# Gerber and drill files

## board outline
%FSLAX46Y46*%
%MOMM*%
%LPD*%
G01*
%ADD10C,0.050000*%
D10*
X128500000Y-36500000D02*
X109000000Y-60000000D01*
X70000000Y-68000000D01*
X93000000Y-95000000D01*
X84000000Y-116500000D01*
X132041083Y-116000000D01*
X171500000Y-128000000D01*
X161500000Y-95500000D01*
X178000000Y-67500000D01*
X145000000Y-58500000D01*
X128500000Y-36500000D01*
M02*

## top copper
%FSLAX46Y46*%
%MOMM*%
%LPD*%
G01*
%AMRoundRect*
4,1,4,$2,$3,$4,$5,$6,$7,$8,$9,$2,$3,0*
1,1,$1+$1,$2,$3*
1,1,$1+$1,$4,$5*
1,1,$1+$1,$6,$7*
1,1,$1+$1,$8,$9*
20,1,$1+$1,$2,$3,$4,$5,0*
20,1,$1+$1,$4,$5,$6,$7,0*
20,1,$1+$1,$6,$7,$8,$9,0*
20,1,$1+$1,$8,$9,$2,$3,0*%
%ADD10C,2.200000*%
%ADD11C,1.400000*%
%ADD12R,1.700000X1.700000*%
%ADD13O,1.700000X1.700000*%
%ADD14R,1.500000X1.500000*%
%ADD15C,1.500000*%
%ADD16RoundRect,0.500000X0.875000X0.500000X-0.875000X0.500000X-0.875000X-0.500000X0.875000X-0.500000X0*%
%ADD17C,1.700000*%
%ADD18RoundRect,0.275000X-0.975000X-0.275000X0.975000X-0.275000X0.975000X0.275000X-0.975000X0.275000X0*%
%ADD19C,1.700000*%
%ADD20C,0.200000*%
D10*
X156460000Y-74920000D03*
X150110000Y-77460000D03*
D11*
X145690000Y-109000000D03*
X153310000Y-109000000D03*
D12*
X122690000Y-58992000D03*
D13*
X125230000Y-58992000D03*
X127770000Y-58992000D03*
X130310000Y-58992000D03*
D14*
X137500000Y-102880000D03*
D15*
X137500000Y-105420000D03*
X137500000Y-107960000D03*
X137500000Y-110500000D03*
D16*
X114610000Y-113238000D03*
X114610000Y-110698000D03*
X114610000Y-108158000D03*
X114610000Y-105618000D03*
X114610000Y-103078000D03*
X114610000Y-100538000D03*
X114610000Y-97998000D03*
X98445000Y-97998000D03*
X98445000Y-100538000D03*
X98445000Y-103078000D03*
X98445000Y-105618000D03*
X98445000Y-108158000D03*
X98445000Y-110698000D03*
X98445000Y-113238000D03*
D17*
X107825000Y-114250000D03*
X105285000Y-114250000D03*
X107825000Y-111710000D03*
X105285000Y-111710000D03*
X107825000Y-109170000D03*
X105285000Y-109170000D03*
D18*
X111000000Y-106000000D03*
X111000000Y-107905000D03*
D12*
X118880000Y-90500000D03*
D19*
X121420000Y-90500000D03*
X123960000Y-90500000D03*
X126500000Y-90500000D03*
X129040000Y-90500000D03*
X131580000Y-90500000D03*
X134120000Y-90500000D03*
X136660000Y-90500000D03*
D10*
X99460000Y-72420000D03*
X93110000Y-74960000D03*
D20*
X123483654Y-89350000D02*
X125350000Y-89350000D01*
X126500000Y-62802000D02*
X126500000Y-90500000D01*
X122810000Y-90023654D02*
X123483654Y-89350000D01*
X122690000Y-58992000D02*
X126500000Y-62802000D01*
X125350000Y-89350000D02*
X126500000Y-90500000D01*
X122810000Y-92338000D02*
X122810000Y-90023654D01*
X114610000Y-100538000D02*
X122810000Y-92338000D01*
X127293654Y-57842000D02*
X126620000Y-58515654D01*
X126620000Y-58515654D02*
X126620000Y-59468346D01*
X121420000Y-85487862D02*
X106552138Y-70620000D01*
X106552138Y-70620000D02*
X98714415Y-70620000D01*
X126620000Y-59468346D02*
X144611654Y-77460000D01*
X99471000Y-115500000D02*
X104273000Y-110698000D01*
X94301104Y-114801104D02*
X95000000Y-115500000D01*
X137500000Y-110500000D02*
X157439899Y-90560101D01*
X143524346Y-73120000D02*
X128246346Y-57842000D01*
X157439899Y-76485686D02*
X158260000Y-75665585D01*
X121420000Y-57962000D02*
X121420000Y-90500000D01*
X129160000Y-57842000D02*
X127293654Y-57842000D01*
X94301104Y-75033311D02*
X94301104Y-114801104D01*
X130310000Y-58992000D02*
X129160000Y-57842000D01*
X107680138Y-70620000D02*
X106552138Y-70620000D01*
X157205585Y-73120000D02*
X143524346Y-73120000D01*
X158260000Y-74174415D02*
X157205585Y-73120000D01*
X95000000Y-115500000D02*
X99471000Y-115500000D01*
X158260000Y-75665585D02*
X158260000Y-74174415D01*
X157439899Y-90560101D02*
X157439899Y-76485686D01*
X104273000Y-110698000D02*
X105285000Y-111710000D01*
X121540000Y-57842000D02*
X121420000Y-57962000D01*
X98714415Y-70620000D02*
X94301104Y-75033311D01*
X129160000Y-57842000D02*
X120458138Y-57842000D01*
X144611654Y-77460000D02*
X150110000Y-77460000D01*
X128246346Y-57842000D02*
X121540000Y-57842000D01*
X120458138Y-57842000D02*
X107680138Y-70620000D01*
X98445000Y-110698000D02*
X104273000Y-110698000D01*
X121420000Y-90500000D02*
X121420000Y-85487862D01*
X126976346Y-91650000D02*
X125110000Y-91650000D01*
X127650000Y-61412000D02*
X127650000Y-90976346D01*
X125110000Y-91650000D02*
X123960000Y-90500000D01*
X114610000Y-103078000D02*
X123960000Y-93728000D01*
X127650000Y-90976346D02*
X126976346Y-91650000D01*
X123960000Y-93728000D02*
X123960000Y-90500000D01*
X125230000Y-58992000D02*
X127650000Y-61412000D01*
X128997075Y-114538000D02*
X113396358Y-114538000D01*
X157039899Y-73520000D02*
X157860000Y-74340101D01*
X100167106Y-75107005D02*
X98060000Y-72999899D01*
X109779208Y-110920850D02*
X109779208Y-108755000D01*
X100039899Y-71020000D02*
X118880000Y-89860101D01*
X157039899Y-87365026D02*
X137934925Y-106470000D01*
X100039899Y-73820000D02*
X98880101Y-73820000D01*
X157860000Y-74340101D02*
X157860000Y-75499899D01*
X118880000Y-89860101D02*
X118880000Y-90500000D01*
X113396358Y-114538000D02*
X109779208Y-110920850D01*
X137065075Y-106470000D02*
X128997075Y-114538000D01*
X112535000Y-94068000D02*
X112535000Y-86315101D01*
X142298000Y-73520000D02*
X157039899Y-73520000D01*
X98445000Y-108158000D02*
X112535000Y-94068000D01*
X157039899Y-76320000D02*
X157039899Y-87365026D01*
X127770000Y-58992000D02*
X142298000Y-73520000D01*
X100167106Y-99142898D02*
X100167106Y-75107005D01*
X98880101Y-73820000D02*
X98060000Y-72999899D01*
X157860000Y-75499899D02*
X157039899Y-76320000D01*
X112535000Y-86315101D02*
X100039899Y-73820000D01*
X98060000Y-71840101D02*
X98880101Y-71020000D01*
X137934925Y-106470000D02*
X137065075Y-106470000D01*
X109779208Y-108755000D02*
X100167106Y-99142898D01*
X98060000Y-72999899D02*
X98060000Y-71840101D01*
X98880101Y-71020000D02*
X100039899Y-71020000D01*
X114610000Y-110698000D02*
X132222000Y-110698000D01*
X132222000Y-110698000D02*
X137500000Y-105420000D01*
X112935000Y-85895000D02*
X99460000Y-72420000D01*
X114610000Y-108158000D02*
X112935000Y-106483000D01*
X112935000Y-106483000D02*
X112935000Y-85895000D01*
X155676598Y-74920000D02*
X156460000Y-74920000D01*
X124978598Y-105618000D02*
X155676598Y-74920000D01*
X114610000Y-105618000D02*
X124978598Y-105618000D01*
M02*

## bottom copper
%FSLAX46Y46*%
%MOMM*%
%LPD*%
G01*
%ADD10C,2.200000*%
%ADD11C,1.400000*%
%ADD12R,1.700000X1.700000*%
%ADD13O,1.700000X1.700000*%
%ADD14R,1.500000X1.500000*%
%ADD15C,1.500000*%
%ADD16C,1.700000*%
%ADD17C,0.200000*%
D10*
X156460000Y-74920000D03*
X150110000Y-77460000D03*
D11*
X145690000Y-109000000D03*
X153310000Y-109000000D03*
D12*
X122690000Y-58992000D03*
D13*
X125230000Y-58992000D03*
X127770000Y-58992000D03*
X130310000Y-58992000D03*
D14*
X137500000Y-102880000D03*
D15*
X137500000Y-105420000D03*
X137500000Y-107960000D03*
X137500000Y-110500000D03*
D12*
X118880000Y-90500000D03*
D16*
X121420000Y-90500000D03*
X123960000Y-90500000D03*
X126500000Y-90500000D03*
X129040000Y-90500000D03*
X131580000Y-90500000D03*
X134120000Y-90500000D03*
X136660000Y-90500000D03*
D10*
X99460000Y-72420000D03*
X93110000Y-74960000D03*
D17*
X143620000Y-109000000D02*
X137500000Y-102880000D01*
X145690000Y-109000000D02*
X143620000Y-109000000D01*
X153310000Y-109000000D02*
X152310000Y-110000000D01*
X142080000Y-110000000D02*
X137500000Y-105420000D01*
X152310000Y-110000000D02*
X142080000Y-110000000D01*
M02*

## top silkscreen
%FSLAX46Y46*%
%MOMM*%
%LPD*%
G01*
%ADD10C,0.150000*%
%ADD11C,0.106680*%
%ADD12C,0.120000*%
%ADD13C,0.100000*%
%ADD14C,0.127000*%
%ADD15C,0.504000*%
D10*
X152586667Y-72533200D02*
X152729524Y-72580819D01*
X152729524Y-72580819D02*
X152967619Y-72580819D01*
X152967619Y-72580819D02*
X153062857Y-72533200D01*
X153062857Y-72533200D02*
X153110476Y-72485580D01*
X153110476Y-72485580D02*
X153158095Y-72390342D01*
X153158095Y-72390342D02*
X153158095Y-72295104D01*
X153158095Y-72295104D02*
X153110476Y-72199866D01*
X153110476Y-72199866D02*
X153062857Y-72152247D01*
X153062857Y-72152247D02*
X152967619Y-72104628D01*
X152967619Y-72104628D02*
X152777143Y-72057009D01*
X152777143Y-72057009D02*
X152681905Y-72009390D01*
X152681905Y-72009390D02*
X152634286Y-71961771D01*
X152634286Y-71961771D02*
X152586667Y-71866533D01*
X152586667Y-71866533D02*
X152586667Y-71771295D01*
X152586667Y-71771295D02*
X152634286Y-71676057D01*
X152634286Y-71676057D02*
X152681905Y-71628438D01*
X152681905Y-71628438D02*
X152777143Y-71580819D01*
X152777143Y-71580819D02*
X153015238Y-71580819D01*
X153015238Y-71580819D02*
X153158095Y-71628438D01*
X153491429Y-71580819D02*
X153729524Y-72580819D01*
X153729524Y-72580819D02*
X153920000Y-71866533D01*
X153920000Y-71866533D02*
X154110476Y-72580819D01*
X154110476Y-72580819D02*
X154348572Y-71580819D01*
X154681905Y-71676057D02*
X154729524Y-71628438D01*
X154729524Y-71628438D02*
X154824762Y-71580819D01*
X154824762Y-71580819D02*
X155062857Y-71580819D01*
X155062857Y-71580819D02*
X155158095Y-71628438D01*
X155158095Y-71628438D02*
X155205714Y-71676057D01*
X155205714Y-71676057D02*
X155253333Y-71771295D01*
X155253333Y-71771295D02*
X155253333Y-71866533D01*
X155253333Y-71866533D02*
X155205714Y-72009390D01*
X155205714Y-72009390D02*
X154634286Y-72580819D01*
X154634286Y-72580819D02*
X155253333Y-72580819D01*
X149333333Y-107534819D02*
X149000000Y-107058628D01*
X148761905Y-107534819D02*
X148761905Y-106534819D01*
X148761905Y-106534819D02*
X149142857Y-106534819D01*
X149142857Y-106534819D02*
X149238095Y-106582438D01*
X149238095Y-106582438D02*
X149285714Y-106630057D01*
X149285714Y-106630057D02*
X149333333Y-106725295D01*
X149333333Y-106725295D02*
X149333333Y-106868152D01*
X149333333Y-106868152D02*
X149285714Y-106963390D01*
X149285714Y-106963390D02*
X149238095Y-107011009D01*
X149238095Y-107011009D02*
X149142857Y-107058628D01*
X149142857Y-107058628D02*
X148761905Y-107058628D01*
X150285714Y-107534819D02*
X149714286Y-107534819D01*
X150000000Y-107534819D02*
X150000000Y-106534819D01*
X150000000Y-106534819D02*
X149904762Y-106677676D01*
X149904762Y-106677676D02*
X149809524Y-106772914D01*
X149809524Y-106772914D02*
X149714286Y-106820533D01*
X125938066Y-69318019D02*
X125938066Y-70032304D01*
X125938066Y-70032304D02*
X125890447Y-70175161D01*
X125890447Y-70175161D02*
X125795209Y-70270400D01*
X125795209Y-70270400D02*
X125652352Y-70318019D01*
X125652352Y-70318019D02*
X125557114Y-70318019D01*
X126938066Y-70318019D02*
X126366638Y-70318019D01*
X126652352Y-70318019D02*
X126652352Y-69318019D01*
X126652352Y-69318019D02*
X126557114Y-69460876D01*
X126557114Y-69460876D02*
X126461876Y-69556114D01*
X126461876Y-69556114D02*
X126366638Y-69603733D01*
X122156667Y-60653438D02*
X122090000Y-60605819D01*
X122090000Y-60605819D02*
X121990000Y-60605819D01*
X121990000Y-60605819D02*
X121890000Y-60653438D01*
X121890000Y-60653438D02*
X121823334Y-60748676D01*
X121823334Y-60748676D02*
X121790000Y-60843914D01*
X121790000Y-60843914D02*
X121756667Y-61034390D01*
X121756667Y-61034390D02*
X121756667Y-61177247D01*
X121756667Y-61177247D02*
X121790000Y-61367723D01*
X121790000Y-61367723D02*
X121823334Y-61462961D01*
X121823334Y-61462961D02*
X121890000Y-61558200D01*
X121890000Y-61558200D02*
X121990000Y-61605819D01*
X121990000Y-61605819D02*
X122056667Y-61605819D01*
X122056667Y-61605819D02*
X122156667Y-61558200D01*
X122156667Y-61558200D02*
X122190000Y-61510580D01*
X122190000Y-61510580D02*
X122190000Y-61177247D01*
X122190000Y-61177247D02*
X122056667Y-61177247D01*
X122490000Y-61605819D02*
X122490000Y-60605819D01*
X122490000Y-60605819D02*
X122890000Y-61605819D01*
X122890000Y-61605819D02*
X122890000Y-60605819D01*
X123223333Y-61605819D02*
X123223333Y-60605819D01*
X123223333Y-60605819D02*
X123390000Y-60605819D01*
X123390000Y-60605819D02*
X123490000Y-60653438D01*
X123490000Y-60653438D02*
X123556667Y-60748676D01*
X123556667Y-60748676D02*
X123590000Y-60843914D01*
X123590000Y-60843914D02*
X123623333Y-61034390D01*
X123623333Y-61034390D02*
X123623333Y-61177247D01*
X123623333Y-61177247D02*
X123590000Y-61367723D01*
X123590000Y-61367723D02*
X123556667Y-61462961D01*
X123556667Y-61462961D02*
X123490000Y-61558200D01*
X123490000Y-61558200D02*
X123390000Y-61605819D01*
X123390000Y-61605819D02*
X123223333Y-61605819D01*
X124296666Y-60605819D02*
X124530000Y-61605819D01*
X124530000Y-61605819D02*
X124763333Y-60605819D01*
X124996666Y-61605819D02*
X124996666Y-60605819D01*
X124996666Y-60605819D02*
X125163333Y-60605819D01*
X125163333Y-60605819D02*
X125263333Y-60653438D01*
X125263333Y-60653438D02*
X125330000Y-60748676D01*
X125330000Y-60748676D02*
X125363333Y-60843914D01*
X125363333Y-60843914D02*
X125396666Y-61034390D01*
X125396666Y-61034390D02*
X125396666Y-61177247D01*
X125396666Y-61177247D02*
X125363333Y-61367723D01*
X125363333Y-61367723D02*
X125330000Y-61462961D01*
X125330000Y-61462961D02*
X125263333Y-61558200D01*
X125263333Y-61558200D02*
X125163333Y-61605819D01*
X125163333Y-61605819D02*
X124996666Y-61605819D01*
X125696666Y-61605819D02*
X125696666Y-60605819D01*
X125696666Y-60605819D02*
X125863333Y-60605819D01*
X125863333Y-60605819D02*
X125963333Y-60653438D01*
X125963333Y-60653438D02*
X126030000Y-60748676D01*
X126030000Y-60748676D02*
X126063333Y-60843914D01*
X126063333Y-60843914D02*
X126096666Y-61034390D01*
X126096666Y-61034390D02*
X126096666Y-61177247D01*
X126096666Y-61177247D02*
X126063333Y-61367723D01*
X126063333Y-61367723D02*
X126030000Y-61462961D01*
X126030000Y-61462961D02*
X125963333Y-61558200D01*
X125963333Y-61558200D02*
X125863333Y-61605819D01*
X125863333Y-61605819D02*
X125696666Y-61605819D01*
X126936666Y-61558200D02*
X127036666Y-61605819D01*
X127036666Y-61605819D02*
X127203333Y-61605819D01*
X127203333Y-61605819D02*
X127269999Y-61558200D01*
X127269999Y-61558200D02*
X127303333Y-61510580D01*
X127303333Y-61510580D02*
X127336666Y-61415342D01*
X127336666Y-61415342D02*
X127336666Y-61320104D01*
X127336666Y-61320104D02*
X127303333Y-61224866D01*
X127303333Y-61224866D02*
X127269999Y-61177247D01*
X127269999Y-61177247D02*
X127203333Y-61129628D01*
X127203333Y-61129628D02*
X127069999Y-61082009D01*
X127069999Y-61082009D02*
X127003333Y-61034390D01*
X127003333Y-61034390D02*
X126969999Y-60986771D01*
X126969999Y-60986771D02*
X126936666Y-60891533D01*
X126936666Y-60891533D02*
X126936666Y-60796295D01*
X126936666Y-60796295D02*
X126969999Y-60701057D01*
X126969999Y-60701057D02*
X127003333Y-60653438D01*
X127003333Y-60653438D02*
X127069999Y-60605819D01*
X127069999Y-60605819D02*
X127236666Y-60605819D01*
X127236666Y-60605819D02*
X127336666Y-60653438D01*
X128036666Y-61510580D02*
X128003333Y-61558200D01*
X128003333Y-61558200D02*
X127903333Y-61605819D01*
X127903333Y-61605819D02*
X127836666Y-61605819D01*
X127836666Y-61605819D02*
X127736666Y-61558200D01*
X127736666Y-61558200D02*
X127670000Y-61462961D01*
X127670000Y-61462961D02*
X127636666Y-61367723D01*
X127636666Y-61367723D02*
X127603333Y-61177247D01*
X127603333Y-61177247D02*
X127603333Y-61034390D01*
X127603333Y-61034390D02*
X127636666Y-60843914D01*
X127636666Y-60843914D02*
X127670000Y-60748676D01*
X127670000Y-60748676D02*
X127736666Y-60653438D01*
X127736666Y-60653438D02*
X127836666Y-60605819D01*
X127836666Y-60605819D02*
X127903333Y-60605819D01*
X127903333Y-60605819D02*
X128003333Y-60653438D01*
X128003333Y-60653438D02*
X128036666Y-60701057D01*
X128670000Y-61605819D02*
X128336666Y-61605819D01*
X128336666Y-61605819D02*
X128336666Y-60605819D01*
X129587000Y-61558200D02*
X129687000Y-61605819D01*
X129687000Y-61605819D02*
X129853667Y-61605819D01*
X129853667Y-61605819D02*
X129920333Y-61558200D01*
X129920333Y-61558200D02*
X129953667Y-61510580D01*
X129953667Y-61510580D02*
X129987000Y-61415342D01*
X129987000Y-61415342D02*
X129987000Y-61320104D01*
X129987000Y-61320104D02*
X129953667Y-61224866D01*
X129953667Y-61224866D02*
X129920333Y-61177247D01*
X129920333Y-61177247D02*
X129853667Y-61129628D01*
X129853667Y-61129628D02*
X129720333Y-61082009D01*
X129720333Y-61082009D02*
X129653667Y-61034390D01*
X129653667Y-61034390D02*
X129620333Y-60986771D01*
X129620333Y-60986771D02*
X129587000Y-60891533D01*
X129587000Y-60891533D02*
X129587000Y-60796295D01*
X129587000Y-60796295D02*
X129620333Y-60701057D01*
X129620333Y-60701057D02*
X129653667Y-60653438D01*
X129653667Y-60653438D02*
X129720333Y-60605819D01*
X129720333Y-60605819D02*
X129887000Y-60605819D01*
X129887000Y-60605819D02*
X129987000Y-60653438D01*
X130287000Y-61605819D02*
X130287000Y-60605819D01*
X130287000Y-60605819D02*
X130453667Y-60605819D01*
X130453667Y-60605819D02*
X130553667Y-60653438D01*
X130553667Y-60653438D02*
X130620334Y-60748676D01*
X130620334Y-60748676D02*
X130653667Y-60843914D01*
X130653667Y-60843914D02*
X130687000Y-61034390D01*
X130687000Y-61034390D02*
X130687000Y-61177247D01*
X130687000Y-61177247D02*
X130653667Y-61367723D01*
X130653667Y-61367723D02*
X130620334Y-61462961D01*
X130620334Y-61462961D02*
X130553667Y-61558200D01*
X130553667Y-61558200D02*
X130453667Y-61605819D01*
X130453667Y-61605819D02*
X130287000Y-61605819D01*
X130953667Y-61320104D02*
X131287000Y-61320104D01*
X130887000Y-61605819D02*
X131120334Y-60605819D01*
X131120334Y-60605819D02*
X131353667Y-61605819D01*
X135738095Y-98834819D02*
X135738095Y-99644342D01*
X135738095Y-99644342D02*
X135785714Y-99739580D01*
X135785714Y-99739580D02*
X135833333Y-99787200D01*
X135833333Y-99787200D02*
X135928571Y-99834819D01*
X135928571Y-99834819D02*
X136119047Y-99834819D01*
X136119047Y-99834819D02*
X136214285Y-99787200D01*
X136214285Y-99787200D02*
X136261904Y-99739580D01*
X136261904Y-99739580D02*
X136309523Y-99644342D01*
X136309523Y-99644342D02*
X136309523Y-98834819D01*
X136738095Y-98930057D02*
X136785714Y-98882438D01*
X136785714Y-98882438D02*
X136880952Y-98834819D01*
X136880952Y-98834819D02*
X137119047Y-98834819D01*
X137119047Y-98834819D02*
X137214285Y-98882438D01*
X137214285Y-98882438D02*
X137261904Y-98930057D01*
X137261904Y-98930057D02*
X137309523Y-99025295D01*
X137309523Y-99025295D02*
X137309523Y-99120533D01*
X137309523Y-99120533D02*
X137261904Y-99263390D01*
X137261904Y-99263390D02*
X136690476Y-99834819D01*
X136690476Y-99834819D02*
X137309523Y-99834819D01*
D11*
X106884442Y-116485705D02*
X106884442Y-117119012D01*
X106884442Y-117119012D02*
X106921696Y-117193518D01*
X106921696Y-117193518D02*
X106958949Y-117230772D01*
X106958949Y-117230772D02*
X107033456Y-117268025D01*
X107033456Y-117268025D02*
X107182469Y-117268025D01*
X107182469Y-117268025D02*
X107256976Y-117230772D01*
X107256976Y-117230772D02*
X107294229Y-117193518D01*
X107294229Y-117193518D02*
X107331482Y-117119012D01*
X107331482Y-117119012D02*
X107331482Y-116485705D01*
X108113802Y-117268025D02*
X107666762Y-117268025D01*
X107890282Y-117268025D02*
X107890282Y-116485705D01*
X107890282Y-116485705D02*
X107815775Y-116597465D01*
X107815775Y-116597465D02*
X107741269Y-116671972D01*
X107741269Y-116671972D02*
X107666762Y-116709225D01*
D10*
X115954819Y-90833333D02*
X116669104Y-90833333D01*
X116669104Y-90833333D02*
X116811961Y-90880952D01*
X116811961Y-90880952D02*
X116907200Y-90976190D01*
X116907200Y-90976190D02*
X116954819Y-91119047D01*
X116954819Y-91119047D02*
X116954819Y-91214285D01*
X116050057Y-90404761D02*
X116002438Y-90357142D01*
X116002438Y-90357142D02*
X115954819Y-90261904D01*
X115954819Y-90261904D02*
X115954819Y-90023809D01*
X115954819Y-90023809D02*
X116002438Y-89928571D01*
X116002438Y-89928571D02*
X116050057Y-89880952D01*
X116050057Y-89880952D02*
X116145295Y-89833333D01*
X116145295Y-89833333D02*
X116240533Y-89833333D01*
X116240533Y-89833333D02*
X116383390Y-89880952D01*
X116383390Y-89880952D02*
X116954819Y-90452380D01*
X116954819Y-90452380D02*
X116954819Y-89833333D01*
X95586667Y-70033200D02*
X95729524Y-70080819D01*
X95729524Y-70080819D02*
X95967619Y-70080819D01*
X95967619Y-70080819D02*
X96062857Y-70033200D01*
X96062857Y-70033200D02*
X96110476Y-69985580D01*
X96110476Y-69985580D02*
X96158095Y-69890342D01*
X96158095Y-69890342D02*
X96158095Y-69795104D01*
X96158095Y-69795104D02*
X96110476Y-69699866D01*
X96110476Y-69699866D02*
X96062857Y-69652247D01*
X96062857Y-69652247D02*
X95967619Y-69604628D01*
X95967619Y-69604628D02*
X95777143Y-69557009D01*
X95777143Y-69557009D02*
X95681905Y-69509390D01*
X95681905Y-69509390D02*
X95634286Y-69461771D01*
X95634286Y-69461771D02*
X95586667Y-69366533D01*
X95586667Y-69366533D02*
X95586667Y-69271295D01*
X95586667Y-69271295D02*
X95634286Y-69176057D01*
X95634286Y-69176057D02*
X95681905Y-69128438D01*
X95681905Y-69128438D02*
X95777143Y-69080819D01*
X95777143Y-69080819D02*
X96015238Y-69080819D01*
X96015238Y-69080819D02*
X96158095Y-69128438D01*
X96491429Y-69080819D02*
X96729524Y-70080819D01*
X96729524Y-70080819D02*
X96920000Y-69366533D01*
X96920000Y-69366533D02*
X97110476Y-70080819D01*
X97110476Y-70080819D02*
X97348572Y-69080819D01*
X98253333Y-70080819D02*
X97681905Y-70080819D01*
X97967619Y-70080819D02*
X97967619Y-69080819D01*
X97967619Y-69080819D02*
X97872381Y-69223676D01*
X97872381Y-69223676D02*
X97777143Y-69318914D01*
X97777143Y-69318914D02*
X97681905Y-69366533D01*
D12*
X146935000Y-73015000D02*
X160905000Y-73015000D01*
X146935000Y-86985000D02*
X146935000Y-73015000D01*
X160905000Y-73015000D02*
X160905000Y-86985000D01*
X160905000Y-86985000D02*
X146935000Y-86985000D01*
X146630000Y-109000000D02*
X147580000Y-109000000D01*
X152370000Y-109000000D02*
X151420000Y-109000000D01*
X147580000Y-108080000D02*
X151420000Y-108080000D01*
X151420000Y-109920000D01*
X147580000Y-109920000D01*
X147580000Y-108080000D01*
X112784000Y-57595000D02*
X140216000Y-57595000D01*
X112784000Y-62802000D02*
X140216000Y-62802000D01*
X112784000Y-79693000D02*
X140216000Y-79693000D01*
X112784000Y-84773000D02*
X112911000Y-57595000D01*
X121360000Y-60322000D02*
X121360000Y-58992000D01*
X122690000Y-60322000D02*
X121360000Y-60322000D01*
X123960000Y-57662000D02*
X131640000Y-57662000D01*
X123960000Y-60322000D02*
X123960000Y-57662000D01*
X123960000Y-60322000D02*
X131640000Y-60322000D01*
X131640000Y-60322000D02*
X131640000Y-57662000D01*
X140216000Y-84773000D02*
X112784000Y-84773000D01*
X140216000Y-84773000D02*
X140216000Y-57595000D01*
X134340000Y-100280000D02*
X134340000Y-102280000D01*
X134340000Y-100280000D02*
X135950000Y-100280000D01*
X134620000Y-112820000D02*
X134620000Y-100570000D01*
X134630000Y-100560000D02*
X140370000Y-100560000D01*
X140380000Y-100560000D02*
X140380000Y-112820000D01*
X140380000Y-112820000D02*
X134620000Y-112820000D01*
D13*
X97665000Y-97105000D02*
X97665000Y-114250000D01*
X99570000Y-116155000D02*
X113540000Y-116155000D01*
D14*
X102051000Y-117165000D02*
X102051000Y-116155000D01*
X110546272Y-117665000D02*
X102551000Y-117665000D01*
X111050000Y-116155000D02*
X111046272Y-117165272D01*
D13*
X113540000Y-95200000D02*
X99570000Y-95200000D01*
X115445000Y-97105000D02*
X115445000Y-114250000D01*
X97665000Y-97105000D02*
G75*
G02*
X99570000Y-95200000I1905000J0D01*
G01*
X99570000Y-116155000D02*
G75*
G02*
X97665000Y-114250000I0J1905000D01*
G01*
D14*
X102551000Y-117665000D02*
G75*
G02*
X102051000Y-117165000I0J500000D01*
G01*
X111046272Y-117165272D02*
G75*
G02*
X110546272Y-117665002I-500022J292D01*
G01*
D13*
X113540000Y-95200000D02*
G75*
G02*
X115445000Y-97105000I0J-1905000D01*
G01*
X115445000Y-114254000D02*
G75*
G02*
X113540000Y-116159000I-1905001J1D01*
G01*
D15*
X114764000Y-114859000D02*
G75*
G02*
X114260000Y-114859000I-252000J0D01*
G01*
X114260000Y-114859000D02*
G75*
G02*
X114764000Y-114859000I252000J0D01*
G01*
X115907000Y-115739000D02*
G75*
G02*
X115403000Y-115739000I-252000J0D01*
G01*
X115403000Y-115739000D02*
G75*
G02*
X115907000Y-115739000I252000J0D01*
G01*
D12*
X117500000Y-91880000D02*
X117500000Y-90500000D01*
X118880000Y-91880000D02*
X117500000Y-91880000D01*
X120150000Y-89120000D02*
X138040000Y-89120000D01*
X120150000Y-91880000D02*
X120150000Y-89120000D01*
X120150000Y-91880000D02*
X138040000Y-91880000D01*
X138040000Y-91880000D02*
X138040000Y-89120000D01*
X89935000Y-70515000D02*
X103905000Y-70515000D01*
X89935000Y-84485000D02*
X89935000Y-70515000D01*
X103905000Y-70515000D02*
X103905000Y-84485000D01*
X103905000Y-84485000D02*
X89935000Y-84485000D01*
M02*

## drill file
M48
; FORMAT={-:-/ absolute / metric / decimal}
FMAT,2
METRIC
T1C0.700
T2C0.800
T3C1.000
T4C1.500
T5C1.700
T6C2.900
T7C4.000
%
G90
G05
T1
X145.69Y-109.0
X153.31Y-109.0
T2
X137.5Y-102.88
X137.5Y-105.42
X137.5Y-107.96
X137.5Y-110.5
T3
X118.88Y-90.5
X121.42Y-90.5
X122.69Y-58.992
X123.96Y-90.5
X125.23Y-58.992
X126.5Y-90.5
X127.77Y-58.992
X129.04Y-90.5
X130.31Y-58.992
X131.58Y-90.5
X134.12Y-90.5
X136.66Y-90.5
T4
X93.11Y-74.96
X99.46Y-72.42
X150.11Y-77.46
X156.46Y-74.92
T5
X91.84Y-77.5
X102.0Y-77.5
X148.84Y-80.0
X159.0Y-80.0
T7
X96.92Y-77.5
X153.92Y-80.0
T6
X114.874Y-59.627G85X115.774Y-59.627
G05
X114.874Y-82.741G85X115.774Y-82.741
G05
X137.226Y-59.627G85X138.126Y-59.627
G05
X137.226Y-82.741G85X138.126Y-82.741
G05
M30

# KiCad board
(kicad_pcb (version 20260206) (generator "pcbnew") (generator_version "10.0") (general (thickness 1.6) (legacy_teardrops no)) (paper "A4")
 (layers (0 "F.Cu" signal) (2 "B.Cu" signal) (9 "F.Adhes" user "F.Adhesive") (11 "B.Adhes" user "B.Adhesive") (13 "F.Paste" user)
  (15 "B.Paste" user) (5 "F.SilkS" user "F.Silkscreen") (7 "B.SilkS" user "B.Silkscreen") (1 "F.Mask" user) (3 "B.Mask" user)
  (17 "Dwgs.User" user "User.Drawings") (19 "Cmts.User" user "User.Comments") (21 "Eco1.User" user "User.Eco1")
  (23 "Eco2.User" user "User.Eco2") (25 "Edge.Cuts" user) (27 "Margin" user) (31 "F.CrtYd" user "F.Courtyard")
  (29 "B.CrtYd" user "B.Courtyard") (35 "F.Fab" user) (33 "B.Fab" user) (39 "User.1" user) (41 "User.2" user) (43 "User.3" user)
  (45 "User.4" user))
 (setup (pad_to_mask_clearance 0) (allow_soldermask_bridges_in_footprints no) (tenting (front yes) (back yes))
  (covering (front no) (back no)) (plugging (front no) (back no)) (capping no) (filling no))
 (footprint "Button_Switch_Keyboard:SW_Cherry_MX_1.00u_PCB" (layer "F.Cu") (at 156.46 74.92)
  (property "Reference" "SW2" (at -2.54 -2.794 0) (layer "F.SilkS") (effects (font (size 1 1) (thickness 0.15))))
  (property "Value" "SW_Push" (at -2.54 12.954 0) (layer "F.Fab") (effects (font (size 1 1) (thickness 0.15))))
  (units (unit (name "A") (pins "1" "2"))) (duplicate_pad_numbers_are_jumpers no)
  (fp_line (start -9.525 -1.905) (end 4.445 -1.905) (stroke (width 0.12) (type solid)) (layer "F.SilkS"))
  (fp_line (start -9.525 12.065) (end -9.525 -1.905) (stroke (width 0.12) (type solid)) (layer "F.SilkS"))
  (fp_line (start 4.445 -1.905) (end 4.445 12.065) (stroke (width 0.12) (type solid)) (layer "F.SilkS"))
  (fp_line (start 4.445 12.065) (end -9.525 12.065) (stroke (width 0.12) (type solid)) (layer "F.SilkS"))
  (pad "" np_thru_hole circle (at -7.62 5.08) (size 1.7 1.7) (drill 1.7) (layers "*.Cu" "*.Mask"))
  (pad "" np_thru_hole circle (at -2.54 5.08) (size 4 4) (drill 4) (layers "*.Cu" "*.Mask"))
  (pad "" np_thru_hole circle (at 2.54 5.08) (size 1.7 1.7) (drill 1.7) (layers "*.Cu" "*.Mask"))
  (pad "1" thru_hole circle (at 0 0) (size 2.2 2.2) (drill 1.5) (layers "*.Cu" "*.Mask") (remove_unused_layers no) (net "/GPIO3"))
  (pad "2" thru_hole circle (at -6.35 2.54) (size 2.2 2.2) (drill 1.5) (layers "*.Cu" "*.Mask") (remove_unused_layers no) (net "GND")))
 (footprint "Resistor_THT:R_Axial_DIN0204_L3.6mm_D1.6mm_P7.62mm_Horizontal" (layer "F.Cu") (at 145.69 109)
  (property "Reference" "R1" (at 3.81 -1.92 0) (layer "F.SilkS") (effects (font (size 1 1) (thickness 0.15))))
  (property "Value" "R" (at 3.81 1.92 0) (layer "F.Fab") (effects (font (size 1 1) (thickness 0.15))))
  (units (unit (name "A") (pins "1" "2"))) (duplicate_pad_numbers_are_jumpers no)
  (fp_line (start 0.94 0) (end 1.89 0) (stroke (width 0.12) (type solid)) (layer "F.SilkS"))
  (fp_line (start 6.68 0) (end 5.73 0) (stroke (width 0.12) (type solid)) (layer "F.SilkS"))
  (fp_rect (start 1.89 -0.92) (end 5.73 0.92) (stroke (width 0.12) (type solid)) (fill no) (layer "F.SilkS"))
  (pad "1" thru_hole circle (at 0 0) (size 1.4 1.4) (drill 0.7) (layers "*.Cu" "*.Mask") (remove_unused_layers no) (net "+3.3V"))
  (pad "2" thru_hole circle (at 7.62 0) (size 1.4 1.4) (drill 0.7) (layers "*.Cu" "*.Mask") (remove_unused_layers no) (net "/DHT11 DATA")))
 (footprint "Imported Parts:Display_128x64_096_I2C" (layer "F.Cu") (at 126.5 58.992)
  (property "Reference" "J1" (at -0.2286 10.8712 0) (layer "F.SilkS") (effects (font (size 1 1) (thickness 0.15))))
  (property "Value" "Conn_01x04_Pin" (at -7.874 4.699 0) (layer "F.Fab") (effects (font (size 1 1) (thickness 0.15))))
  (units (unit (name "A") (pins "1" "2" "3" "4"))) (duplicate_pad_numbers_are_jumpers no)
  (fp_line (start -13.716 -1.397) (end 13.716 -1.397) (stroke (width 0.12) (type solid)) (layer "F.SilkS"))
  (fp_line (start -13.716 3.81) (end 13.716 3.81) (stroke (width 0.12) (type solid)) (layer "F.SilkS"))
  (fp_line (start -13.716 20.701) (end 13.716 20.701) (stroke (width 0.12) (type solid)) (layer "F.SilkS"))
  (fp_line (start -13.716 25.781) (end -13.589 -1.397) (stroke (width 0.12) (type solid)) (layer "F.SilkS"))
  (fp_line (start -5.14 1.33) (end -5.14 0) (stroke (width 0.12) (type solid)) (layer "F.SilkS"))
  (fp_line (start -3.81 1.33) (end -5.14 1.33) (stroke (width 0.12) (type solid)) (layer "F.SilkS"))
  (fp_line (start -2.54 -1.33) (end 5.14 -1.33) (stroke (width 0.12) (type solid)) (layer "F.SilkS"))
  (fp_line (start -2.54 1.33) (end -2.54 -1.33) (stroke (width 0.12) (type solid)) (layer "F.SilkS"))
  (fp_line (start -2.54 1.33) (end 5.14 1.33) (stroke (width 0.12) (type solid)) (layer "F.SilkS"))
  (fp_line (start 5.14 1.33) (end 5.14 -1.33) (stroke (width 0.12) (type solid)) (layer "F.SilkS"))
  (fp_line (start 13.716 25.781) (end -13.716 25.781) (stroke (width 0.12) (type solid)) (layer "F.SilkS"))
  (fp_line (start 13.716 25.781) (end 13.716 -1.397) (stroke (width 0.12) (type solid)) (layer "F.SilkS"))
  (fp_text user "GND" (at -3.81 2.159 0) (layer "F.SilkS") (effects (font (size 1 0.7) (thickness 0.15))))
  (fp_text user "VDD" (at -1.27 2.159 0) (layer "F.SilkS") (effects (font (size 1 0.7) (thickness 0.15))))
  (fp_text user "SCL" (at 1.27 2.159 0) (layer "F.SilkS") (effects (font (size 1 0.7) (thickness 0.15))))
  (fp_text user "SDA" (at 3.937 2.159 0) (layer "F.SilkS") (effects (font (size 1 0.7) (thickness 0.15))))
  (pad "" np_thru_hole oval (at -11.176 0.635) (size 3.8 2.9) (drill oval 3.8 2.9) (layers "*.Cu" "*.Mask"))
  (pad "" np_thru_hole oval (at -11.176 23.749) (size 3.8 2.9) (drill oval 3.8 2.9) (layers "*.Cu" "*.Mask"))
  (pad "" np_thru_hole oval (at 11.176 0.635) (size 3.8 2.9) (drill oval 3.8 2.9) (layers "*.Cu" "*.Mask"))
  (pad "" np_thru_hole oval (at 11.176 23.749) (size 3.8 2.9) (drill oval 3.8 2.9) (layers "*.Cu" "*.Mask"))
  (pad "1" thru_hole rect (at -3.81 0 90) (size 1.7 1.7) (drill 1) (layers "*.Cu" "*.Mask") (remove_unused_layers no) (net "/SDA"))
  (pad "2" thru_hole oval (at -1.27 0 90) (size 1.7 1.7) (drill 1) (layers "*.Cu" "*.Mask") (remove_unused_layers no) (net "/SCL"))
  (pad "3" thru_hole oval (at 1.27 0 90) (size 1.7 1.7) (drill 1) (layers "*.Cu" "*.Mask") (remove_unused_layers no) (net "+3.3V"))
  (pad "4" thru_hole oval (at 3.81 0 90) (size 1.7 1.7) (drill 1) (layers "*.Cu" "*.Mask") (remove_unused_layers no) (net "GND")))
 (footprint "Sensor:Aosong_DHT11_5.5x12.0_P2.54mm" (layer "F.Cu") (at 137.5 102.88)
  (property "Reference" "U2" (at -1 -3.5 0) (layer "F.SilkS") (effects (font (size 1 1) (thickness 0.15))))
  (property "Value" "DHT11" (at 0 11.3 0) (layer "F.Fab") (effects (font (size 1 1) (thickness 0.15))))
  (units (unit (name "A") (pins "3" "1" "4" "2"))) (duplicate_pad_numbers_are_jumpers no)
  (fp_line (start -3.16 -2.6) (end -3.16 -0.6) (stroke (width 0.12) (type solid)) (layer "F.SilkS"))
  (fp_line (start -3.16 -2.6) (end -1.55 -2.6) (stroke (width 0.12) (type solid)) (layer "F.SilkS"))
  (fp_line (start -2.88 9.94) (end -2.88 -2.31) (stroke (width 0.12) (type solid)) (layer "F.SilkS"))
  (fp_line (start -2.87 -2.32) (end 2.87 -2.32) (stroke (width 0.12) (type solid)) (layer "F.SilkS"))
  (fp_line (start 2.88 -2.32) (end 2.88 9.94) (stroke (width 0.12) (type solid)) (layer "F.SilkS"))
  (fp_line (start 2.88 9.94) (end -2.88 9.94) (stroke (width 0.12) (type solid)) (layer "F.SilkS"))
  (pad "1" thru_hole rect (at 0 0) (size 1.5 1.5) (drill 0.8) (layers "*.Cu" "*.Mask") (remove_unused_layers no) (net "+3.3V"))
  (pad "2" thru_hole circle (at 0 2.54) (size 1.5 1.5) (drill 0.8) (layers "*.Cu" "*.Mask") (remove_unused_layers no) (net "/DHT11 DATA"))
  (pad "3" thru_hole circle (at 0 5.08) (size 1.5 1.5) (drill 0.8) (layers "*.Cu" "*.Mask") (remove_unused_layers no)
   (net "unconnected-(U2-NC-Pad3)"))
  (pad "4" thru_hole circle (at 0 7.62) (size 1.5 1.5) (drill 0.8) (layers "*.Cu" "*.Mask") (remove_unused_layers no) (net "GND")))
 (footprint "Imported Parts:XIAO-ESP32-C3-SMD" (layer "F.Cu") (at 115.445 95.118 180)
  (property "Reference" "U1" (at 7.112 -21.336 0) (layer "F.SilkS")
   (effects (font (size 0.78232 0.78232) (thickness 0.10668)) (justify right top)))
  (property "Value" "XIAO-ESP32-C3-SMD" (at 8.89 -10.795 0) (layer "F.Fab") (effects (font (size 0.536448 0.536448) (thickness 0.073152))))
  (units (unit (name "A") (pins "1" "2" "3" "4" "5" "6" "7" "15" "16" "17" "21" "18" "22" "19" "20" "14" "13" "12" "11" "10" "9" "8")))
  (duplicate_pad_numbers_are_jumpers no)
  (fp_line (start 17.78 -1.987) (end 17.78 -19.132) (stroke (width 0.1) (type solid)) (layer "F.SilkS"))
  (fp_line (start 15.875 -21.037) (end 1.905 -21.037) (stroke (width 0.1) (type solid)) (layer "F.SilkS"))
  (fp_line (start 13.394 -22.047) (end 13.394 -21.037) (stroke (width 0.127) (type solid)) (layer "F.SilkS"))
  (fp_line (start 4.898728 -22.547) (end 12.894 -22.547) (stroke (width 0.127) (type solid)) (layer "F.SilkS"))
  (fp_line (start 4.395 -21.037) (end 4.398728 -22.047272) (stroke (width 0.127) (type solid)) (layer "F.SilkS"))
  (fp_line (start 1.905 -0.082) (end 15.875 -0.082) (stroke (width 0.1) (type solid)) (layer "F.SilkS"))
  (fp_line (start 0 -1.987) (end 0 -19.132) (stroke (width 0.1) (type solid)) (layer "F.SilkS"))
  (fp_arc (start 17.78 -1.987) (mid 17.222038 -0.639962) (end 15.875 -0.082) (stroke (width 0.1) (type solid)) (layer "F.SilkS"))
  (fp_arc (start 15.875 -21.037) (mid 17.222038 -20.479038) (end 17.78 -19.132) (stroke (width 0.1) (type solid)) (layer "F.SilkS"))
  (fp_arc (start 12.894 -22.547) (mid 13.247553 -22.400553) (end 13.394 -22.047) (stroke (width 0.127) (type default)) (layer "F.SilkS"))
  (fp_arc (start 4.398728 -22.047272) (mid 4.545272 -22.40064) (end 4.898728 -22.547) (stroke (width 0.127) (type default))
   (layer "F.SilkS"))
  (fp_arc (start 1.905 -0.082) (mid 0.557962 -0.639962) (end 0 -1.987) (stroke (width 0.1) (type solid)) (layer "F.SilkS"))
  (fp_arc (start 0 -19.136) (mid 0.557962 -20.483038) (end 1.905 -21.041) (stroke (width 0.1) (type solid)) (layer "F.SilkS"))
  (fp_circle (center 0.933 -19.741) (end 0.933 -19.995) (stroke (width 0.5) (type solid)) (fill yes) (layer "F.SilkS"))
  (fp_circle (center -0.21 -20.621) (end -0.21 -20.875) (stroke (width 0.5) (type solid)) (fill yes) (layer "F.SilkS"))
  (pad "1" smd roundrect (at 0.835 -18.12 180) (size 2.75 2) (layers "F.Cu" "F.Mask" "F.Paste") (roundrect_rratio 0.25)
   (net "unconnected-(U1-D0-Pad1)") (solder_mask_margin 0.0508) (thermal_bridge_angle 45))
  (pad "2" smd roundrect (at 0.835 -15.58 180) (size 2.75 2) (layers "F.Cu" "F.Mask" "F.Paste") (roundrect_rratio 0.25) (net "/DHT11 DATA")
   (solder_mask_margin 0.0508) (thermal_bridge_angle 45))
  (pad "3" smd roundrect (at 0.835 -13.04 180) (size 2.75 2) (layers "F.Cu" "F.Mask" "F.Paste") (roundrect_rratio 0.25) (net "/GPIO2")
   (solder_mask_margin 0.0508) (thermal_bridge_angle 45))
  (pad "4" smd roundrect (at 0.835 -10.5 180) (size 2.75 2) (layers "F.Cu" "F.Mask" "F.Paste") (roundrect_rratio 0.25) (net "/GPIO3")
   (solder_mask_margin 0.0508) (thermal_bridge_angle 45))
  (pad "5" smd roundrect (at 0.835 -7.96 180) (size 2.75 2) (layers "F.Cu" "F.Mask" "F.Paste") (roundrect_rratio 0.25) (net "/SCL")
   (solder_mask_margin 0.0508) (thermal_bridge_angle 45))
  (pad "6" smd roundrect (at 0.835 -5.42 180) (size 2.75 2) (layers "F.Cu" "F.Mask" "F.Paste") (roundrect_rratio 0.25) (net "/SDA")
   (solder_mask_margin 0.0508) (thermal_bridge_angle 45))
  (pad "7" smd roundrect (at 0.835 -2.88 180) (size 2.75 2) (layers "F.Cu" "F.Mask" "F.Paste") (roundrect_rratio 0.25)
   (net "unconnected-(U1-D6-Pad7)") (solder_mask_margin 0.0508) (thermal_bridge_angle 45))
  (pad "8" smd roundrect (at 17 -2.88 180) (size 2.75 2) (layers "F.Cu" "F.Mask" "F.Paste") (roundrect_rratio 0.25)
   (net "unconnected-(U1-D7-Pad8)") (solder_mask_margin 0.0508) (thermal_bridge_angle 45))
  (pad "9" smd roundrect (at 17 -5.42 180) (size 2.75 2) (layers "F.Cu" "F.Mask" "F.Paste") (roundrect_rratio 0.25)
   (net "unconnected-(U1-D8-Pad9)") (solder_mask_margin 0.0508) (thermal_bridge_angle 45))
  (pad "10" smd roundrect (at 17 -7.96 180) (size 2.75 2) (layers "F.Cu" "F.Mask" "F.Paste") (roundrect_rratio 0.25)
   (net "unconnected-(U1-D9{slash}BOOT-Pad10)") (solder_mask_margin 0.0508) (thermal_bridge_angle 45))
  (pad "11" smd roundrect (at 17 -10.5 180) (size 2.75 2) (layers "F.Cu" "F.Mask" "F.Paste") (roundrect_rratio 0.25)
   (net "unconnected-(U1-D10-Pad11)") (solder_mask_margin 0.0508) (thermal_bridge_angle 45))
  (pad "12" smd roundrect (at 17 -13.04 180) (size 2.75 2) (layers "F.Cu" "F.Mask" "F.Paste") (roundrect_rratio 0.25) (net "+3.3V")
   (solder_mask_margin 0.0508) (thermal_bridge_angle 45))
  (pad "13" smd roundrect (at 17 -15.58 180) (size 2.75 2) (layers "F.Cu" "F.Mask" "F.Paste") (roundrect_rratio 0.25) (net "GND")
   (solder_mask_margin 0.0508) (thermal_bridge_angle 45))
  (pad "14" smd roundrect (at 17 -18.12 180) (size 2.75 2) (layers "F.Cu" "F.Mask" "F.Paste") (roundrect_rratio 0.25) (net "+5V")
   (solder_mask_margin 0.0508) (thermal_bridge_angle 45))
  (pad "15" smd circle (at 7.62 -19.132 180) (size 1.7 1.7) (layers "F.Cu" "F.Mask" "F.Paste") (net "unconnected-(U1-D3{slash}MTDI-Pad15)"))
  (pad "16" smd circle (at 10.16 -19.132 180) (size 1.7 1.7) (layers "F.Cu" "F.Mask" "F.Paste") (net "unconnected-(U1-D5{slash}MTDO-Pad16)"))
  (pad "17" smd circle (at 7.62 -16.592 180) (size 1.7 1.7) (layers "F.Cu" "F.Mask" "F.Paste") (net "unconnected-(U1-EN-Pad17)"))
  (pad "18" smd circle (at 10.16 -16.592 180) (size 1.7 1.7) (layers "F.Cu" "F.Mask" "F.Paste") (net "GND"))
  (pad "19" smd circle (at 7.62 -14.052 180) (size 1.7 1.7) (layers "F.Cu" "F.Mask" "F.Paste") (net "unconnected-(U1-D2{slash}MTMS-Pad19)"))
  (pad "20" smd circle (at 10.16 -14.052 180) (size 1.7 1.7) (layers "F.Cu" "F.Mask" "F.Paste") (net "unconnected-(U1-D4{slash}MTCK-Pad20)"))
  (pad "21" smd roundrect (at 4.445 -10.882) (size 2.5 1.1) (layers "F.Cu" "F.Mask" "F.Paste") (roundrect_rratio 0.25)
   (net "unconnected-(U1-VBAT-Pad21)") (thermal_bridge_angle 45))
  (pad "22" smd roundrect (at 4.445 -12.787) (size 2.5 1.1) (layers "F.Cu" "F.Mask" "F.Paste") (roundrect_rratio 0.25)
   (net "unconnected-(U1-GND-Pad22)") (thermal_bridge_angle 45)))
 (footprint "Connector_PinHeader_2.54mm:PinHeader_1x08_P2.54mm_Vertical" (layer "F.Cu") (at 118.88 90.5 90)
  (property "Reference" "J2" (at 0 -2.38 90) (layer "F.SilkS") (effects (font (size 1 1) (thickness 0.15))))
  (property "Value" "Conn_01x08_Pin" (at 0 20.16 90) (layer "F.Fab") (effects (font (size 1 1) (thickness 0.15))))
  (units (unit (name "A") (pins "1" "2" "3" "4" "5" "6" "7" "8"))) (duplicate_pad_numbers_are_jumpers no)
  (fp_line (start -1.38 -1.38) (end 0 -1.38) (stroke (width 0.12) (type solid)) (layer "F.SilkS"))
  (fp_line (start -1.38 0) (end -1.38 -1.38) (stroke (width 0.12) (type solid)) (layer "F.SilkS"))
  (fp_line (start 1.38 1.27) (end 1.38 19.16) (stroke (width 0.12) (type solid)) (layer "F.SilkS"))
  (fp_line (start -1.38 1.27) (end 1.38 1.27) (stroke (width 0.12) (type solid)) (layer "F.SilkS"))
  (fp_line (start -1.38 1.27) (end -1.38 19.16) (stroke (width 0.12) (type solid)) (layer "F.SilkS"))
  (fp_line (start -1.38 19.16) (end 1.38 19.16) (stroke (width 0.12) (type solid)) (layer "F.SilkS"))
  (pad "1" thru_hole rect (at 0 0 90) (size 1.7 1.7) (drill 1) (layers "*.Cu" "*.Mask") (remove_unused_layers no) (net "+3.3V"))
  (pad "2" thru_hole circle (at 0 2.54 90) (size 1.7 1.7) (drill 1) (layers "*.Cu" "*.Mask") (remove_unused_layers no) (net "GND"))
  (pad "3" thru_hole circle (at 0 5.08 90) (size 1.7 1.7) (drill 1) (layers "*.Cu" "*.Mask") (remove_unused_layers no) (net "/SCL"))
  (pad "4" thru_hole circle (at 0 7.62 90) (size 1.7 1.7) (drill 1) (layers "*.Cu" "*.Mask") (remove_unused_layers no) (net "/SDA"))
  (pad "5" thru_hole circle (at 0 10.16 90) (size 1.7 1.7) (drill 1) (layers "*.Cu" "*.Mask") (remove_unused_layers no)
   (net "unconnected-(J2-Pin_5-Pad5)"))
  (pad "6" thru_hole circle (at 0 12.7 90) (size 1.7 1.7) (drill 1) (layers "*.Cu" "*.Mask") (remove_unused_layers no)
   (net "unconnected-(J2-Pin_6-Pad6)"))
  (pad "7" thru_hole circle (at 0 15.24 90) (size 1.7 1.7) (drill 1) (layers "*.Cu" "*.Mask") (remove_unused_layers no)
   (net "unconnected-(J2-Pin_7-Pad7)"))
  (pad "8" thru_hole circle (at 0 17.78 90) (size 1.7 1.7) (drill 1) (layers "*.Cu" "*.Mask") (remove_unused_layers no)
   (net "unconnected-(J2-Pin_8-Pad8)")))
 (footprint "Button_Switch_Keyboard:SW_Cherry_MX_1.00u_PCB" (layer "F.Cu") (at 99.46 72.42)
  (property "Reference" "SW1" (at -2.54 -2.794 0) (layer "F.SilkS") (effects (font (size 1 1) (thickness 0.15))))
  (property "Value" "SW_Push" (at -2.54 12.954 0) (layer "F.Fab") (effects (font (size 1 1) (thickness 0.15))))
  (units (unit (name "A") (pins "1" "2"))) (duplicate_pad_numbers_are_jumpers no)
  (fp_line (start -9.525 -1.905) (end 4.445 -1.905) (stroke (width 0.12) (type solid)) (layer "F.SilkS"))
  (fp_line (start -9.525 12.065) (end -9.525 -1.905) (stroke (width 0.12) (type solid)) (layer "F.SilkS"))
  (fp_line (start 4.445 -1.905) (end 4.445 12.065) (stroke (width 0.12) (type solid)) (layer "F.SilkS"))
  (fp_line (start 4.445 12.065) (end -9.525 12.065) (stroke (width 0.12) (type solid)) (layer "F.SilkS"))
  (pad "" np_thru_hole circle (at -7.62 5.08) (size 1.7 1.7) (drill 1.7) (layers "*.Cu" "*.Mask"))
  (pad "" np_thru_hole circle (at -2.54 5.08) (size 4 4) (drill 4) (layers "*.Cu" "*.Mask"))
  (pad "" np_thru_hole circle (at 2.54 5.08) (size 1.7 1.7) (drill 1.7) (layers "*.Cu" "*.Mask"))
  (pad "1" thru_hole circle (at 0 0) (size 2.2 2.2) (drill 1.5) (layers "*.Cu" "*.Mask") (remove_unused_layers no) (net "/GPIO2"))
  (pad "2" thru_hole circle (at -6.35 2.54) (size 2.2 2.2) (drill 1.5) (layers "*.Cu" "*.Mask") (remove_unused_layers no) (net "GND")))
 (gr_poly
  (pts (xy 128.5 36.5) (xy 109 60) (xy 70 68) (xy 93 95) (xy 84 116.5) (xy 132.041083 116) (xy 171.5 128) (xy 161.5 95.5) (xy 178 67.5)
   (xy 145 58.5))
  (stroke (width 0.05) (type solid)) (fill no) (layer "Edge.Cuts"))
 (segment (start 123.483654 89.35) (end 125.35 89.35) (width 0.2) (layer "F.Cu") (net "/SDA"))
 (segment (start 126.5 62.802) (end 126.5 90.5) (width 0.2) (layer "F.Cu") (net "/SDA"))
 (segment (start 122.81 90.023654) (end 123.483654 89.35) (width 0.2) (layer "F.Cu") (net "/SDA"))
 (segment (start 122.69 58.992) (end 126.5 62.802) (width 0.2) (layer "F.Cu") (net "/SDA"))
 (segment (start 125.35 89.35) (end 126.5 90.5) (width 0.2) (layer "F.Cu") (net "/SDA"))
 (segment (start 122.81 92.338) (end 122.81 90.023654) (width 0.2) (layer "F.Cu") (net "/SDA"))
 (segment (start 114.61 100.538) (end 122.81 92.338) (width 0.2) (layer "F.Cu") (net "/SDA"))
 (segment (start 127.293654 57.842) (end 126.62 58.515654) (width 0.2) (layer "F.Cu") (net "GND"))
 (segment (start 126.62 58.515654) (end 126.62 59.468346) (width 0.2) (layer "F.Cu") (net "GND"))
 (segment (start 121.42 85.487862) (end 106.552138 70.62) (width 0.2) (layer "F.Cu") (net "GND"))
 (segment (start 106.552138 70.62) (end 98.714415 70.62) (width 0.2) (layer "F.Cu") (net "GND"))
 (segment (start 126.62 59.468346) (end 144.611654 77.46) (width 0.2) (layer "F.Cu") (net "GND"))
 (segment (start 99.471 115.5) (end 104.273 110.698) (width 0.2) (layer "F.Cu") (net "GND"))
 (segment (start 94.301104 114.801104) (end 95 115.5) (width 0.2) (layer "F.Cu") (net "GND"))
 (segment (start 137.5 110.5) (end 157.439899 90.560101) (width 0.2) (layer "F.Cu") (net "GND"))
 (segment (start 143.524346 73.12) (end 128.246346 57.842) (width 0.2) (layer "F.Cu") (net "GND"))
 (segment (start 157.439899 76.485686) (end 158.26 75.665585) (width 0.2) (layer "F.Cu") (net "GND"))
 (segment (start 121.42 57.962) (end 121.42 90.5) (width 0.2) (layer "F.Cu") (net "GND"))
 (segment (start 129.16 57.842) (end 127.293654 57.842) (width 0.2) (layer "F.Cu") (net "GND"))
 (segment (start 94.301104 75.033311) (end 94.301104 114.801104) (width 0.2) (layer "F.Cu") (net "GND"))
 (segment (start 130.31 58.992) (end 129.16 57.842) (width 0.2) (layer "F.Cu") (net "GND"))
 (segment (start 107.680138 70.62) (end 106.552138 70.62) (width 0.2) (layer "F.Cu") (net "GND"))
 (segment (start 157.205585 73.12) (end 143.524346 73.12) (width 0.2) (layer "F.Cu") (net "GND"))
 (segment (start 158.26 74.174415) (end 157.205585 73.12) (width 0.2) (layer "F.Cu") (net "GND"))
 (segment (start 95 115.5) (end 99.471 115.5) (width 0.2) (layer "F.Cu") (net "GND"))
 (segment (start 158.26 75.665585) (end 158.26 74.174415) (width 0.2) (layer "F.Cu") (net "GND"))
 (segment (start 157.439899 90.560101) (end 157.439899 76.485686) (width 0.2) (layer "F.Cu") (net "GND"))
 (segment (start 104.273 110.698) (end 105.285 111.71) (width 0.2) (layer "F.Cu") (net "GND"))
 (segment (start 121.54 57.842) (end 121.42 57.962) (width 0.2) (layer "F.Cu") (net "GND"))
 (segment (start 98.714415 70.62) (end 94.301104 75.033311) (width 0.2) (layer "F.Cu") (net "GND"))
 (segment (start 129.16 57.842) (end 120.458138 57.842) (width 0.2) (layer "F.Cu") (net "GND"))
 (segment (start 144.611654 77.46) (end 150.11 77.46) (width 0.2) (layer "F.Cu") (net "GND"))
 (segment (start 128.246346 57.842) (end 121.54 57.842) (width 0.2) (layer "F.Cu") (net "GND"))
 (segment (start 120.458138 57.842) (end 107.680138 70.62) (width 0.2) (layer "F.Cu") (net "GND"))
 (segment (start 98.445 110.698) (end 104.273 110.698) (width 0.2) (layer "F.Cu") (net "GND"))
 (segment (start 121.42 90.5) (end 121.42 85.487862) (width 0.2) (layer "F.Cu") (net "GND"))
 (segment (start 126.976346 91.65) (end 125.11 91.65) (width 0.2) (layer "F.Cu") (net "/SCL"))
 (segment (start 127.65 61.412) (end 127.65 90.976346) (width 0.2) (layer "F.Cu") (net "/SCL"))
 (segment (start 125.11 91.65) (end 123.96 90.5) (width 0.2) (layer "F.Cu") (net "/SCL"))
 (segment (start 114.61 103.078) (end 123.96 93.728) (width 0.2) (layer "F.Cu") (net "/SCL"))
 (segment (start 127.65 90.976346) (end 126.976346 91.65) (width 0.2) (layer "F.Cu") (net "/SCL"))
 (segment (start 123.96 93.728) (end 123.96 90.5) (width 0.2) (layer "F.Cu") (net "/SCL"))
 (segment (start 125.23 58.992) (end 127.65 61.412) (width 0.2) (layer "F.Cu") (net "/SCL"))
 (segment (start 128.997075 114.538) (end 113.396358 114.538) (width 0.2) (layer "F.Cu") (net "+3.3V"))
 (segment (start 157.039899 73.52) (end 157.86 74.340101) (width 0.2) (layer "F.Cu") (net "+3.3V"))
 (segment (start 100.167106 75.107005) (end 98.06 72.999899) (width 0.2) (layer "F.Cu") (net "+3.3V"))
 (segment (start 109.779208 110.92085) (end 109.779208 108.755) (width 0.2) (layer "F.Cu") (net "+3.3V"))
 (segment (start 100.039899 71.02) (end 118.88 89.860101) (width 0.2) (layer "F.Cu") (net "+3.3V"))
 (segment (start 157.039899 87.365026) (end 137.934925 106.47) (width 0.2) (layer "F.Cu") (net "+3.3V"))
 (segment (start 100.039899 73.82) (end 98.880101 73.82) (width 0.2) (layer "F.Cu") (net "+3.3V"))
 (segment (start 157.86 74.340101) (end 157.86 75.499899) (width 0.2) (layer "F.Cu") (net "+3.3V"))
 (segment (start 118.88 89.860101) (end 118.88 90.5) (width 0.2) (layer "F.Cu") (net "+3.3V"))
 (segment (start 113.396358 114.538) (end 109.779208 110.92085) (width 0.2) (layer "F.Cu") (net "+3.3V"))
 (segment (start 137.065075 106.47) (end 128.997075 114.538) (width 0.2) (layer "F.Cu") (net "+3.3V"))
 (segment (start 112.535 94.068) (end 112.535 86.315101) (width 0.2) (layer "F.Cu") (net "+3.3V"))
 (segment (start 142.298 73.52) (end 157.039899 73.52) (width 0.2) (layer "F.Cu") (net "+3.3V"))
 (segment (start 98.445 108.158) (end 112.535 94.068) (width 0.2) (layer "F.Cu") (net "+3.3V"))
 (segment (start 157.039899 76.32) (end 157.039899 87.365026) (width 0.2) (layer "F.Cu") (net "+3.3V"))
 (segment (start 127.77 58.992) (end 142.298 73.52) (width 0.2) (layer "F.Cu") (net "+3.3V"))
 (segment (start 100.167106 99.142898) (end 100.167106 75.107005) (width 0.2) (layer "F.Cu") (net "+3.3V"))
 (segment (start 98.880101 73.82) (end 98.06 72.999899) (width 0.2) (layer "F.Cu") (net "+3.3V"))
 (segment (start 157.86 75.499899) (end 157.039899 76.32) (width 0.2) (layer "F.Cu") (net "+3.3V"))
 (segment (start 112.535 86.315101) (end 100.039899 73.82) (width 0.2) (layer "F.Cu") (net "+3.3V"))
 (segment (start 98.06 71.840101) (end 98.880101 71.02) (width 0.2) (layer "F.Cu") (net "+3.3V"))
 (segment (start 137.934925 106.47) (end 137.065075 106.47) (width 0.2) (layer "F.Cu") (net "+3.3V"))
 (segment (start 109.779208 108.755) (end 100.167106 99.142898) (width 0.2) (layer "F.Cu") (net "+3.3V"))
 (segment (start 98.06 72.999899) (end 98.06 71.840101) (width 0.2) (layer "F.Cu") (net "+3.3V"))
 (segment (start 98.880101 71.02) (end 100.039899 71.02) (width 0.2) (layer "F.Cu") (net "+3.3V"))
 (segment (start 143.62 109) (end 137.5 102.88) (width 0.2) (layer "B.Cu") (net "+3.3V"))
 (segment (start 145.69 109) (end 143.62 109) (width 0.2) (layer "B.Cu") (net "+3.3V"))
 (segment (start 114.61 110.698) (end 132.222 110.698) (width 0.2) (layer "F.Cu") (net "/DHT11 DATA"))
 (segment (start 132.222 110.698) (end 137.5 105.42) (width 0.2) (layer "F.Cu") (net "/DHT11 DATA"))
 (segment (start 153.31 109) (end 152.31 110) (width 0.2) (layer "B.Cu") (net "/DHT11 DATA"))
 (segment (start 142.08 110) (end 137.5 105.42) (width 0.2) (layer "B.Cu") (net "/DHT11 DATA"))
 (segment (start 152.31 110) (end 142.08 110) (width 0.2) (layer "B.Cu") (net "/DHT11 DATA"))
 (segment (start 112.935 85.895) (end 99.46 72.42) (width 0.2) (layer "F.Cu") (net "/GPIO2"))
 (segment (start 114.61 108.158) (end 112.935 106.483) (width 0.2) (layer "F.Cu") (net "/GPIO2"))
 (segment (start 112.935 106.483) (end 112.935 85.895) (width 0.2) (layer "F.Cu") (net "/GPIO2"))
 (segment (start 155.676598 74.92) (end 156.46 74.92) (width 0.2) (layer "F.Cu") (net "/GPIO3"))
 (segment (start 124.978598 105.618) (end 155.676598 74.92) (width 0.2) (layer "F.Cu") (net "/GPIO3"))
 (segment (start 114.61 105.618) (end 124.978598 105.618) (width 0.2) (layer "F.Cu") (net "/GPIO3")))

